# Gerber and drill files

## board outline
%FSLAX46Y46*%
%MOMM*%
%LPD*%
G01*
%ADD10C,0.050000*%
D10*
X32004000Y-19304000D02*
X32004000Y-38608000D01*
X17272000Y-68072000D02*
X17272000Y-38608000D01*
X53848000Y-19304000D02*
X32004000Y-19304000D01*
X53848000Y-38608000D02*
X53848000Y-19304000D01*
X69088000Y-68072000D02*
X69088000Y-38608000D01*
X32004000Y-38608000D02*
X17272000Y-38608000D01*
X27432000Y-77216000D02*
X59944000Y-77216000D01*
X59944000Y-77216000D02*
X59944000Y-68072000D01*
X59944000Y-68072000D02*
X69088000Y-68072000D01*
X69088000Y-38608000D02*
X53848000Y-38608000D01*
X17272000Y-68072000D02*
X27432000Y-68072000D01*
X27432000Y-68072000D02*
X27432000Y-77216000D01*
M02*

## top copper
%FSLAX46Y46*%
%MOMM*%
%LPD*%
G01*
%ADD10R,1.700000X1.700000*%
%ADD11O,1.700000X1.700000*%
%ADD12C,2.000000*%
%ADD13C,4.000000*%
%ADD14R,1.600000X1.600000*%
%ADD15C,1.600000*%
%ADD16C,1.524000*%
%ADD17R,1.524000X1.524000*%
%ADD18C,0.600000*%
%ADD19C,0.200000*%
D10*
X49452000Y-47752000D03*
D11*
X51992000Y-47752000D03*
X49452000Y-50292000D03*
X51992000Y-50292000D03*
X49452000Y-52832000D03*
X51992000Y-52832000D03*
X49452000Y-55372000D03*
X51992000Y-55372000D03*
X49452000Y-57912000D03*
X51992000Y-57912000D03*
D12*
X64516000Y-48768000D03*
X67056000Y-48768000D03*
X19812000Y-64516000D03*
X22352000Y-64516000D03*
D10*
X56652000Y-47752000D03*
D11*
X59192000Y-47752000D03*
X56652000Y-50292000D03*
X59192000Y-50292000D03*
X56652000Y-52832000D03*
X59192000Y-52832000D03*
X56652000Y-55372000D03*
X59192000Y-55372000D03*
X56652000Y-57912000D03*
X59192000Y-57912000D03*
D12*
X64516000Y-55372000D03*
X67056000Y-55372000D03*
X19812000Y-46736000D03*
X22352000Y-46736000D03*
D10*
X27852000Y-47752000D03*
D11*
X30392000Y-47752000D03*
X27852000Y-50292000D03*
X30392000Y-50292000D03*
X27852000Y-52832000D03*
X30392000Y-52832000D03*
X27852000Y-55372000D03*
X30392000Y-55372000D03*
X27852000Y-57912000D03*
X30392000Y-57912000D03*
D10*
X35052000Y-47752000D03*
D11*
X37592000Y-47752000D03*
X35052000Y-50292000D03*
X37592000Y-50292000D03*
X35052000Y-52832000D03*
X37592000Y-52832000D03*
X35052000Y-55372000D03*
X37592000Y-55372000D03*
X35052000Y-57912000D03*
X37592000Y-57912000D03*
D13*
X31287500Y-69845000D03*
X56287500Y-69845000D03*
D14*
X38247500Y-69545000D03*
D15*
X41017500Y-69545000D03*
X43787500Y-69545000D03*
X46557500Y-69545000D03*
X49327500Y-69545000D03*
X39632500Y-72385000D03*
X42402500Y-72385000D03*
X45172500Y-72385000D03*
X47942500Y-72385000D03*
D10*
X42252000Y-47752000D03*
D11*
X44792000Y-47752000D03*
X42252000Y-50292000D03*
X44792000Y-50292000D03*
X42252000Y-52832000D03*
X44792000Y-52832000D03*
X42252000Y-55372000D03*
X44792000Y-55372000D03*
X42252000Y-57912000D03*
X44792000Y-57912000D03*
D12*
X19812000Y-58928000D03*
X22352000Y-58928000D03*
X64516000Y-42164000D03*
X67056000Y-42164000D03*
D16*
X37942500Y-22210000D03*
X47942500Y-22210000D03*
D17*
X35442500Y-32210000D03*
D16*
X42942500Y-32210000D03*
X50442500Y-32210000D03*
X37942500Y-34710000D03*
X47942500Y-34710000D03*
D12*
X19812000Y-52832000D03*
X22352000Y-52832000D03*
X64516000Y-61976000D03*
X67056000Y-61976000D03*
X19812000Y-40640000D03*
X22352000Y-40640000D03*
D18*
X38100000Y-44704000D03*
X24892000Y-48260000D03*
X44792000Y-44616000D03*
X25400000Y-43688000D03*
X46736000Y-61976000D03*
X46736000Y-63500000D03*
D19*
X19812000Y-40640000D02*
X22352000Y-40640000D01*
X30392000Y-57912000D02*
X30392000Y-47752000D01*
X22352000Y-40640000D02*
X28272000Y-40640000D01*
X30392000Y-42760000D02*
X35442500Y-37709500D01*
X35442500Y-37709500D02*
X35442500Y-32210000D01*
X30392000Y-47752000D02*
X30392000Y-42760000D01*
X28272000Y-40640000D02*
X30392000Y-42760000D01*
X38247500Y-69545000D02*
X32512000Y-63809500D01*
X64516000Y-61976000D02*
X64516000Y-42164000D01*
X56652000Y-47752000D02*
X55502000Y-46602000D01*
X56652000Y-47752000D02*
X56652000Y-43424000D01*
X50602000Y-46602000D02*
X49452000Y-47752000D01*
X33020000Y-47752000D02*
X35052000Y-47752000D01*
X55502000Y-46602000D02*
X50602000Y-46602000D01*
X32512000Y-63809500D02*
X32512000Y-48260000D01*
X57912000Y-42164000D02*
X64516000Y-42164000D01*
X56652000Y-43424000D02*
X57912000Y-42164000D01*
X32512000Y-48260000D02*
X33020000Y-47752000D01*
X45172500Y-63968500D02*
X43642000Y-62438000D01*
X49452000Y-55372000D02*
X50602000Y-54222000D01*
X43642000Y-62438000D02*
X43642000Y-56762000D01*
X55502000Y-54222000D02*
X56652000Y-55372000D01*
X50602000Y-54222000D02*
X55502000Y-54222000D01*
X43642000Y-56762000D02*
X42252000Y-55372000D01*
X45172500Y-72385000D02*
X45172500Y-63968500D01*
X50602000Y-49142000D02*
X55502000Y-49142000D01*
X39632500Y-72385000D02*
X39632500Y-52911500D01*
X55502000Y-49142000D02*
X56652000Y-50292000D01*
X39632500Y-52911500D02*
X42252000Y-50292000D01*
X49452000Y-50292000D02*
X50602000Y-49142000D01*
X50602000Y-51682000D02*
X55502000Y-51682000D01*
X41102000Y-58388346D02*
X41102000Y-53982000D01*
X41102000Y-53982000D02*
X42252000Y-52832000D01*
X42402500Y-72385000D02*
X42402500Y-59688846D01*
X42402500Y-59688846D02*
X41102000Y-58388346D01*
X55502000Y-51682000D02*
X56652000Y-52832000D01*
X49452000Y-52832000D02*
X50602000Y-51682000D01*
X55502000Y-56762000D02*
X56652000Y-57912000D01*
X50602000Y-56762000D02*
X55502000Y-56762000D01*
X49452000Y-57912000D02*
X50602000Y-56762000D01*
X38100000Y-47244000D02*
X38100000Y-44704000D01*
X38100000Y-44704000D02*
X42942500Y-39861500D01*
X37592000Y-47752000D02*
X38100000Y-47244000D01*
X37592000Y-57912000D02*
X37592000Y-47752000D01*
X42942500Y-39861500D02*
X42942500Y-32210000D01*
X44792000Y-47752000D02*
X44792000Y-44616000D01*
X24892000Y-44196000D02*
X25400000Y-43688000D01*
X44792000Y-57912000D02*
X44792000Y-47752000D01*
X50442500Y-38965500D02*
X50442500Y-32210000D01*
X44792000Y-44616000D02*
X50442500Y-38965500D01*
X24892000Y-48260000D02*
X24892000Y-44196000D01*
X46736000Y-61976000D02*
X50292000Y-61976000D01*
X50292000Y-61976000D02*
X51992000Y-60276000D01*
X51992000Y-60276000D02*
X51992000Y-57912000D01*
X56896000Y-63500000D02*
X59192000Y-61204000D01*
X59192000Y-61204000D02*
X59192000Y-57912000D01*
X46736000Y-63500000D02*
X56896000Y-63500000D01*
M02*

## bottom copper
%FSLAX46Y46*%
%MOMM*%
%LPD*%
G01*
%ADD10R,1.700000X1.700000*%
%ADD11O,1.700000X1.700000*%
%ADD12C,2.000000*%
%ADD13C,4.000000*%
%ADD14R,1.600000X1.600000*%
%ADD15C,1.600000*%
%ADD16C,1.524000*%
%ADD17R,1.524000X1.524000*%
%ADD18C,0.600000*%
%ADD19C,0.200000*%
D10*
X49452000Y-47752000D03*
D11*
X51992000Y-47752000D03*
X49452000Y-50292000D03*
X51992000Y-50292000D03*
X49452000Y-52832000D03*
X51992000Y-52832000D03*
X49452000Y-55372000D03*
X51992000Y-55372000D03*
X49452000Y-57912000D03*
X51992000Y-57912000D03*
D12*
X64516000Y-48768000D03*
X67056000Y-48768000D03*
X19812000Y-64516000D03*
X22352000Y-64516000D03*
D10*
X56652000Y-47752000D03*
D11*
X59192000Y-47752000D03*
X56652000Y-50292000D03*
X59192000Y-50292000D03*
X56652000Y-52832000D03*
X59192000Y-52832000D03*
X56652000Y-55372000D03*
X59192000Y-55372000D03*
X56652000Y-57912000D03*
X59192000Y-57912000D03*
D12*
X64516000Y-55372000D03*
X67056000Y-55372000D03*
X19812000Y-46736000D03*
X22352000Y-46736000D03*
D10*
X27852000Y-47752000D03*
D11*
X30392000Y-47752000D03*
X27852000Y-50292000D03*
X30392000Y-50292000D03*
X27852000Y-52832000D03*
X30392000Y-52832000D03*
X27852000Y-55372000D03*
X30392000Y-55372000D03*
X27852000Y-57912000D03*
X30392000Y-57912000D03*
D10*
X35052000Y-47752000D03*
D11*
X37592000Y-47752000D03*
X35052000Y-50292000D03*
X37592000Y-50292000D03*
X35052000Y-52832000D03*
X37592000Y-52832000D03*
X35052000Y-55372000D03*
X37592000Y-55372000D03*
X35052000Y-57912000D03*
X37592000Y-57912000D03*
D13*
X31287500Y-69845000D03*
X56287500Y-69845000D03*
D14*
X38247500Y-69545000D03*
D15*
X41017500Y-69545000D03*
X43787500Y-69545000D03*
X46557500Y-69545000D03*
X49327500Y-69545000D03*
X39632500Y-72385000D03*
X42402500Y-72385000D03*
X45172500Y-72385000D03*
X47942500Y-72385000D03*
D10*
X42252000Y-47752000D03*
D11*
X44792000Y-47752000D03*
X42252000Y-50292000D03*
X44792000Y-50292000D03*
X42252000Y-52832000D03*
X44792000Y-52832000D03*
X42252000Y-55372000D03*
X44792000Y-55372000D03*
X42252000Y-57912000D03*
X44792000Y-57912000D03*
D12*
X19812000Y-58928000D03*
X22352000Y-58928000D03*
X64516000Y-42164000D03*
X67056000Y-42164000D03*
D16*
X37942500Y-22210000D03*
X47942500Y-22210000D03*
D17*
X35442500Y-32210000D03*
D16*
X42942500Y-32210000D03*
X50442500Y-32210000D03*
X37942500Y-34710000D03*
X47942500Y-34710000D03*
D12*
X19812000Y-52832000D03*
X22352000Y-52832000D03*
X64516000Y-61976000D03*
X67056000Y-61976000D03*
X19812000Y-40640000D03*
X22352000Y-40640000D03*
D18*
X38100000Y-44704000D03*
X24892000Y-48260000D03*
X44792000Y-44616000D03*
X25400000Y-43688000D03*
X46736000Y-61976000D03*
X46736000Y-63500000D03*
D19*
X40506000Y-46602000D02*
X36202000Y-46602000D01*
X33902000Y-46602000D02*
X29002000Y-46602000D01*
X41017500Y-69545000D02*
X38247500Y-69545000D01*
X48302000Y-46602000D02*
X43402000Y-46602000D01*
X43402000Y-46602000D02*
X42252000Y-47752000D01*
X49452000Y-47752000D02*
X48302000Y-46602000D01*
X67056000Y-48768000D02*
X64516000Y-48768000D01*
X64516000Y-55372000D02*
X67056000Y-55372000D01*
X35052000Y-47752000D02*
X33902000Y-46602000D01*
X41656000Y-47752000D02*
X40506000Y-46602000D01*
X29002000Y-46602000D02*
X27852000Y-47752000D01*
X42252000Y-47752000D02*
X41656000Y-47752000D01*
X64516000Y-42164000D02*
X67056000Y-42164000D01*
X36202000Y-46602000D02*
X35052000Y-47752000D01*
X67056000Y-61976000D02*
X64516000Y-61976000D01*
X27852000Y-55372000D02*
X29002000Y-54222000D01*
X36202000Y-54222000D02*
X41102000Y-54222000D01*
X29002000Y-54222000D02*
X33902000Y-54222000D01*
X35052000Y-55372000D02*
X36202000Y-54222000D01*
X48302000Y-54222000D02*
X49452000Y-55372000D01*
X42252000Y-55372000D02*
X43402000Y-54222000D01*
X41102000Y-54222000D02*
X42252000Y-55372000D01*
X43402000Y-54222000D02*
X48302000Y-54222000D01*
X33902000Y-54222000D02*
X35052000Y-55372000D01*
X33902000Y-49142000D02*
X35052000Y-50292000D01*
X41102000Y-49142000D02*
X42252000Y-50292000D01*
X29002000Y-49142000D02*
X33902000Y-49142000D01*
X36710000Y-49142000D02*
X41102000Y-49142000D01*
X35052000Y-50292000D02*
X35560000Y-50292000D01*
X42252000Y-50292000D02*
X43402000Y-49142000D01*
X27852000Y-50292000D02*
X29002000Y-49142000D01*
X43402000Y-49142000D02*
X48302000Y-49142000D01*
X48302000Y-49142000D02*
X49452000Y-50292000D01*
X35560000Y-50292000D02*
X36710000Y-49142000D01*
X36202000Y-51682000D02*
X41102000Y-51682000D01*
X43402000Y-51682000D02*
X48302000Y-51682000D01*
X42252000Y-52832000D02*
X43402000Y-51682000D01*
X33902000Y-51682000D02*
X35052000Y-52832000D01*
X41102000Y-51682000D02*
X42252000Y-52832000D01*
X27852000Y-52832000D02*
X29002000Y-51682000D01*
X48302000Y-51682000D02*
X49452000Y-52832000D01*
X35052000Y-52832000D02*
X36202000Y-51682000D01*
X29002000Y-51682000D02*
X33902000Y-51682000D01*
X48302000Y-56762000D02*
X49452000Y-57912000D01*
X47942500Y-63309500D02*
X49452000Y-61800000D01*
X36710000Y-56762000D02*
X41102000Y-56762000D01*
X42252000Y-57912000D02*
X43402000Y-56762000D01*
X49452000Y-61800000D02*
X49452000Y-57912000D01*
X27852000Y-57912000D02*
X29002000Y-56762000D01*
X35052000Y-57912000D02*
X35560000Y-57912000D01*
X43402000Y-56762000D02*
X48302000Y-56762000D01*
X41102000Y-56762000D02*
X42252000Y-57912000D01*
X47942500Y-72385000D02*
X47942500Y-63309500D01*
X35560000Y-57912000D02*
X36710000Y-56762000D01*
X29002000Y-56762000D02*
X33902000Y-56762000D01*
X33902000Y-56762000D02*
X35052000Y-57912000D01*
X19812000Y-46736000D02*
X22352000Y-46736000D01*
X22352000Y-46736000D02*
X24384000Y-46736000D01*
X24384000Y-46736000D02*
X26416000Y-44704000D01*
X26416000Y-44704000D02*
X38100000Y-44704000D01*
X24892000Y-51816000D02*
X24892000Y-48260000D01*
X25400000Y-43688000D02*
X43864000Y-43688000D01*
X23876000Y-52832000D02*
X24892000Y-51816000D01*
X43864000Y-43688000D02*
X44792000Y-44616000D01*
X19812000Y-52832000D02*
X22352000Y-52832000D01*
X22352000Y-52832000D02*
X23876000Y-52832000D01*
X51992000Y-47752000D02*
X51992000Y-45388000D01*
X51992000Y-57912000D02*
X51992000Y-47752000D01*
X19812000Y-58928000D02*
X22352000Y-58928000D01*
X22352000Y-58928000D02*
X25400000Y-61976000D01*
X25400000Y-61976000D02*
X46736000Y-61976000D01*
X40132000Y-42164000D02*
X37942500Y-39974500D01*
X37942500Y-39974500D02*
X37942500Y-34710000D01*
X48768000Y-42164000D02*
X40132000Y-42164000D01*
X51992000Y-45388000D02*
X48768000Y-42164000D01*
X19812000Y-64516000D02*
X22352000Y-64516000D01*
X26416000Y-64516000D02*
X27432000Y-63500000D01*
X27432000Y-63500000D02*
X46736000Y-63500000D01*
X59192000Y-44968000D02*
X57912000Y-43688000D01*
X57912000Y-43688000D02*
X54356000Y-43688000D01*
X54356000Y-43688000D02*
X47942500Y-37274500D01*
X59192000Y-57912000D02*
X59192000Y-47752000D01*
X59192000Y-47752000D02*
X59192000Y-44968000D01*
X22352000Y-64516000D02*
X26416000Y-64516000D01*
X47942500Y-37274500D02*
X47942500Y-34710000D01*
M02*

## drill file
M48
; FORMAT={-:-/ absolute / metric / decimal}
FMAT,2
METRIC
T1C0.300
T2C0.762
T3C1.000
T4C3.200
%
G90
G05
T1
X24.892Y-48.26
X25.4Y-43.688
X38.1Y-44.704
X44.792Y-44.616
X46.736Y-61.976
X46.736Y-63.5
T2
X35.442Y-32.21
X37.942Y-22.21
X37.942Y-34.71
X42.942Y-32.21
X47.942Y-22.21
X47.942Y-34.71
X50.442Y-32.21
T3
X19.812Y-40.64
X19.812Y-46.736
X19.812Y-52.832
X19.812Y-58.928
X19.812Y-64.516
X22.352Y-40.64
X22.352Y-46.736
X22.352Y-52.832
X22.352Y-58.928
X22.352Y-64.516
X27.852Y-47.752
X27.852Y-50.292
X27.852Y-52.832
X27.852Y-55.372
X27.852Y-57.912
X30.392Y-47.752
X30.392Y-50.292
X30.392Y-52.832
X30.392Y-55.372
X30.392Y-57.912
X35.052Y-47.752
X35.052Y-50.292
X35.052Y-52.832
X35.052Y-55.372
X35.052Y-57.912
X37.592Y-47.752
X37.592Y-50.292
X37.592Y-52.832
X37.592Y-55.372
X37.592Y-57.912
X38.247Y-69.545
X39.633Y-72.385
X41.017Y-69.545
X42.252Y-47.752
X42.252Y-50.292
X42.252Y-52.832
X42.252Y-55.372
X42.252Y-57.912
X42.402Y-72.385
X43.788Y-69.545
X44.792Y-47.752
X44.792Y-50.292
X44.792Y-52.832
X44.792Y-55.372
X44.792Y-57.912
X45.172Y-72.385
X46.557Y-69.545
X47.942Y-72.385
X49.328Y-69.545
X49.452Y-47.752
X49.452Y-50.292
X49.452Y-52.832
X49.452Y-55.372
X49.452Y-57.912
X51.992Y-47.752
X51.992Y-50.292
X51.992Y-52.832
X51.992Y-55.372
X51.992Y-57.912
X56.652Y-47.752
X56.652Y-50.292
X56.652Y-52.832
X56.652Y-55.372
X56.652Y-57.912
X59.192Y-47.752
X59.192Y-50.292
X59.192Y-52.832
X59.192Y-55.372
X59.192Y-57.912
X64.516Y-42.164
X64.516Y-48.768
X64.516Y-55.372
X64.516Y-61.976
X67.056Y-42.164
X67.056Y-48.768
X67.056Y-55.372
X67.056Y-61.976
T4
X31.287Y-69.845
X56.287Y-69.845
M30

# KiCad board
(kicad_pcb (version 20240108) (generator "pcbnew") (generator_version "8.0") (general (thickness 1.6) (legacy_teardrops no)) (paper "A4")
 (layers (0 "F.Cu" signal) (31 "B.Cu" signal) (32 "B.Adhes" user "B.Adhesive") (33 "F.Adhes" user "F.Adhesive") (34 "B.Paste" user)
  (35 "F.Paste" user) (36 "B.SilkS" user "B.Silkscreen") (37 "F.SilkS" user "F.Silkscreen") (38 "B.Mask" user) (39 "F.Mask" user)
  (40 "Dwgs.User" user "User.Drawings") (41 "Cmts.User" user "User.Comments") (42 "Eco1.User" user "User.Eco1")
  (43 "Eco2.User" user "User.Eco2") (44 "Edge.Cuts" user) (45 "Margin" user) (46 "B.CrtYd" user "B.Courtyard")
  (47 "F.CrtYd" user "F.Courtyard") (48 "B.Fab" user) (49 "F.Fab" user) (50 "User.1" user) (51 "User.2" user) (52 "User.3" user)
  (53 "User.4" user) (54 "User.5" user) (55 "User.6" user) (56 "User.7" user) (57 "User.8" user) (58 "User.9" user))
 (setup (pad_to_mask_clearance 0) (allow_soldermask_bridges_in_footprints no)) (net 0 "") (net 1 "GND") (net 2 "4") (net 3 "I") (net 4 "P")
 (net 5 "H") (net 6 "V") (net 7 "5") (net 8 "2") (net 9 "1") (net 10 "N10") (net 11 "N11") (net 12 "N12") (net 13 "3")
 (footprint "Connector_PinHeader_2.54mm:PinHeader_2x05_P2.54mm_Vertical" (layer "F.Cu") (at 49.452 47.752)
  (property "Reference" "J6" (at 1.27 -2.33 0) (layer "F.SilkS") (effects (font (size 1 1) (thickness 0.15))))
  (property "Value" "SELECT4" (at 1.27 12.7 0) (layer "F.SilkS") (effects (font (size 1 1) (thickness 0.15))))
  (pad "1" thru_hole rect (at 0 0) (size 1.7 1.7) (drill 1) (layers "*.Cu" "*.Mask") (remove_unused_layers no) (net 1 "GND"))
  (pad "2" thru_hole oval (at 2.54 0) (size 1.7 1.7) (drill 1) (layers "*.Cu" "*.Mask") (remove_unused_layers no) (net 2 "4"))
  (pad "3" thru_hole oval (at 0 2.54) (size 1.7 1.7) (drill 1) (layers "*.Cu" "*.Mask") (remove_unused_layers no) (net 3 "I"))
  (pad "4" thru_hole oval (at 2.54 2.54) (size 1.7 1.7) (drill 1) (layers "*.Cu" "*.Mask") (remove_unused_layers no) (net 2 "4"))
  (pad "5" thru_hole oval (at 0 5.08) (size 1.7 1.7) (drill 1) (layers "*.Cu" "*.Mask") (remove_unused_layers no) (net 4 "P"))
  (pad "6" thru_hole oval (at 2.54 5.08) (size 1.7 1.7) (drill 1) (layers "*.Cu" "*.Mask") (remove_unused_layers no) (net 2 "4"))
  (pad "7" thru_hole oval (at 0 7.62) (size 1.7 1.7) (drill 1) (layers "*.Cu" "*.Mask") (remove_unused_layers no) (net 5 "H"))
  (pad "8" thru_hole oval (at 2.54 7.62) (size 1.7 1.7) (drill 1) (layers "*.Cu" "*.Mask") (remove_unused_layers no) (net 2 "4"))
  (pad "9" thru_hole oval (at 0 10.16) (size 1.7 1.7) (drill 1) (layers "*.Cu" "*.Mask") (remove_unused_layers no) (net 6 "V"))
  (pad "10" thru_hole oval (at 2.54 10.16) (size 1.7 1.7) (drill 1) (layers "*.Cu" "*.Mask") (remove_unused_layers no) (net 2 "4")))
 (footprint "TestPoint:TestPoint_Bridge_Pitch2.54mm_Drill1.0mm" (layer "F.Cu") (at 64.516 48.768)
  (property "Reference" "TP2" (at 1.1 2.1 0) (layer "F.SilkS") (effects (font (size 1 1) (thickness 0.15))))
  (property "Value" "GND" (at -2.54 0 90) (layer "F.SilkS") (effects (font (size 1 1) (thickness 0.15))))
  (pad "1" thru_hole circle (at 0 0) (size 2 2) (drill 1) (layers "*.Cu" "*.Mask") (remove_unused_layers no) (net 1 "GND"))
  (pad "1" thru_hole circle (at 2.54 0) (size 2 2) (drill 1) (layers "*.Cu" "*.Mask") (remove_unused_layers no) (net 1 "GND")))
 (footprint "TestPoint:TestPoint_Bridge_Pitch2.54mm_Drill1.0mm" (layer "F.Cu") (at 19.812 64.516)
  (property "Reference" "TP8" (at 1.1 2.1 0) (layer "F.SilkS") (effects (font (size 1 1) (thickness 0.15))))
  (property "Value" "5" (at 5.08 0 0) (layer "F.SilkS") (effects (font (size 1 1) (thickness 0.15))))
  (pad "1" thru_hole circle (at 0 0) (size 2 2) (drill 1) (layers "*.Cu" "*.Mask") (remove_unused_layers no) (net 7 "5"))
  (pad "1" thru_hole circle (at 2.54 0) (size 2 2) (drill 1) (layers "*.Cu" "*.Mask") (remove_unused_layers no) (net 7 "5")))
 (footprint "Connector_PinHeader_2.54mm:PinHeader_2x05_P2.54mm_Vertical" (layer "F.Cu") (at 56.652 47.752)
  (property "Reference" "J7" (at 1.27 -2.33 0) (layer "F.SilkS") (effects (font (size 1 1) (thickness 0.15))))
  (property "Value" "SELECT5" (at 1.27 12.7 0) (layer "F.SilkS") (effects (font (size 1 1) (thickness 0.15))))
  (pad "1" thru_hole rect (at 0 0) (size 1.7 1.7) (drill 1) (layers "*.Cu" "*.Mask") (remove_unused_layers no) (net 1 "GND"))
  (pad "2" thru_hole oval (at 2.54 0) (size 1.7 1.7) (drill 1) (layers "*.Cu" "*.Mask") (remove_unused_layers no) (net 7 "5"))
  (pad "3" thru_hole oval (at 0 2.54) (size 1.7 1.7) (drill 1) (layers "*.Cu" "*.Mask") (remove_unused_layers no) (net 3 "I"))
  (pad "4" thru_hole oval (at 2.54 2.54) (size 1.7 1.7) (drill 1) (layers "*.Cu" "*.Mask") (remove_unused_layers no) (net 7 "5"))
  (pad "5" thru_hole oval (at 0 5.08) (size 1.7 1.7) (drill 1) (layers "*.Cu" "*.Mask") (remove_unused_layers no) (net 4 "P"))
  (pad "6" thru_hole oval (at 2.54 5.08) (size 1.7 1.7) (drill 1) (layers "*.Cu" "*.Mask") (remove_unused_layers no) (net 7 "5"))
  (pad "7" thru_hole oval (at 0 7.62) (size 1.7 1.7) (drill 1) (layers "*.Cu" "*.Mask") (remove_unused_layers no) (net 5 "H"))
  (pad "8" thru_hole oval (at 2.54 7.62) (size 1.7 1.7) (drill 1) (layers "*.Cu" "*.Mask") (remove_unused_layers no) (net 7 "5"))
  (pad "9" thru_hole oval (at 0 10.16) (size 1.7 1.7) (drill 1) (layers "*.Cu" "*.Mask") (remove_unused_layers no) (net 6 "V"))
  (pad "10" thru_hole oval (at 2.54 10.16) (size 1.7 1.7) (drill 1) (layers "*.Cu" "*.Mask") (remove_unused_layers no) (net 7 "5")))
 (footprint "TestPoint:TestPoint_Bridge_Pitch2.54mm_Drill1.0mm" (layer "F.Cu") (at 64.516 55.372)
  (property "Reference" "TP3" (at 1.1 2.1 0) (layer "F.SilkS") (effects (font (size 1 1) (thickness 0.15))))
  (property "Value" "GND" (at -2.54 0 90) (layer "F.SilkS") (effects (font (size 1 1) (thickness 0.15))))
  (pad "1" thru_hole circle (at 0 0) (size 2 2) (drill 1) (layers "*.Cu" "*.Mask") (remove_unused_layers no) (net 1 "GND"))
  (pad "1" thru_hole circle (at 2.54 0) (size 2 2) (drill 1) (layers "*.Cu" "*.Mask") (remove_unused_layers no) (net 1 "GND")))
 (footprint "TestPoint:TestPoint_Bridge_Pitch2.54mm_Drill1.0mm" (layer "F.Cu") (at 19.812 46.736)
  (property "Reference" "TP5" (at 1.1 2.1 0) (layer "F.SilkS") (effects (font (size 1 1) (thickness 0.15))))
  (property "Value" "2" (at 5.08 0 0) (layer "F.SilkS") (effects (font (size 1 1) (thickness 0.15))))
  (pad "1" thru_hole circle (at 0 0) (size 2 2) (drill 1) (layers "*.Cu" "*.Mask") (remove_unused_layers no) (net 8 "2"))
  (pad "1" thru_hole circle (at 2.54 0) (size 2 2) (drill 1) (layers "*.Cu" "*.Mask") (remove_unused_layers no) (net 8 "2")))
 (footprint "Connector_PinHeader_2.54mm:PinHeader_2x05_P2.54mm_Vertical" (layer "F.Cu") (at 27.852 47.752)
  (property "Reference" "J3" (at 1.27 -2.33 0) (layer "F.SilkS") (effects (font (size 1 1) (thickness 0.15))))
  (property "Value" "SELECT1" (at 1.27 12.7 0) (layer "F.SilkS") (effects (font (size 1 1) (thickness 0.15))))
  (pad "1" thru_hole rect (at 0 0) (size 1.7 1.7) (drill 1) (layers "*.Cu" "*.Mask") (remove_unused_layers no) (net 1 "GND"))
  (pad "2" thru_hole oval (at 2.54 0) (size 1.7 1.7) (drill 1) (layers "*.Cu" "*.Mask") (remove_unused_layers no) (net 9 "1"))
  (pad "3" thru_hole oval (at 0 2.54) (size 1.7 1.7) (drill 1) (layers "*.Cu" "*.Mask") (remove_unused_layers no) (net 3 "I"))
  (pad "4" thru_hole oval (at 2.54 2.54) (size 1.7 1.7) (drill 1) (layers "*.Cu" "*.Mask") (remove_unused_layers no) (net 9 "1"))
  (pad "5" thru_hole oval (at 0 5.08) (size 1.7 1.7) (drill 1) (layers "*.Cu" "*.Mask") (remove_unused_layers no) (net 4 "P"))
  (pad "6" thru_hole oval (at 2.54 5.08) (size 1.7 1.7) (drill 1) (layers "*.Cu" "*.Mask") (remove_unused_layers no) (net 9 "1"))
  (pad "7" thru_hole oval (at 0 7.62) (size 1.7 1.7) (drill 1) (layers "*.Cu" "*.Mask") (remove_unused_layers no) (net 5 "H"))
  (pad "8" thru_hole oval (at 2.54 7.62) (size 1.7 1.7) (drill 1) (layers "*.Cu" "*.Mask") (remove_unused_layers no) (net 9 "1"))
  (pad "9" thru_hole oval (at 0 10.16) (size 1.7 1.7) (drill 1) (layers "*.Cu" "*.Mask") (remove_unused_layers no) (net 6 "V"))
  (pad "10" thru_hole oval (at 2.54 10.16) (size 1.7 1.7) (drill 1) (layers "*.Cu" "*.Mask") (remove_unused_layers no) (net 9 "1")))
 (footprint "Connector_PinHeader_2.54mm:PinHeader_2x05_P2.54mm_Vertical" (layer "F.Cu") (at 35.052 47.752)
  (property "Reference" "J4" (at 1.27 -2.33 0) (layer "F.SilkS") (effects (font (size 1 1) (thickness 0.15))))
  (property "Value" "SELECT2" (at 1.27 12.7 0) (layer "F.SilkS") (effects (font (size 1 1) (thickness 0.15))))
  (pad "1" thru_hole rect (at 0 0) (size 1.7 1.7) (drill 1) (layers "*.Cu" "*.Mask") (remove_unused_layers no) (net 1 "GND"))
  (pad "2" thru_hole oval (at 2.54 0) (size 1.7 1.7) (drill 1) (layers "*.Cu" "*.Mask") (remove_unused_layers no) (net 8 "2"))
  (pad "3" thru_hole oval (at 0 2.54) (size 1.7 1.7) (drill 1) (layers "*.Cu" "*.Mask") (remove_unused_layers no) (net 3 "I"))
  (pad "4" thru_hole oval (at 2.54 2.54) (size 1.7 1.7) (drill 1) (layers "*.Cu" "*.Mask") (remove_unused_layers no) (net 8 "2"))
  (pad "5" thru_hole oval (at 0 5.08) (size 1.7 1.7) (drill 1) (layers "*.Cu" "*.Mask") (remove_unused_layers no) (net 4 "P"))
  (pad "6" thru_hole oval (at 2.54 5.08) (size 1.7 1.7) (drill 1) (layers "*.Cu" "*.Mask") (remove_unused_layers no) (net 8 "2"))
  (pad "7" thru_hole oval (at 0 7.62) (size 1.7 1.7) (drill 1) (layers "*.Cu" "*.Mask") (remove_unused_layers no) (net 5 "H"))
  (pad "8" thru_hole oval (at 2.54 7.62) (size 1.7 1.7) (drill 1) (layers "*.Cu" "*.Mask") (remove_unused_layers no) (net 8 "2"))
  (pad "9" thru_hole oval (at 0 10.16) (size 1.7 1.7) (drill 1) (layers "*.Cu" "*.Mask") (remove_unused_layers no) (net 6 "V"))
  (pad "10" thru_hole oval (at 2.54 10.16) (size 1.7 1.7) (drill 1) (layers "*.Cu" "*.Mask") (remove_unused_layers no) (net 8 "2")))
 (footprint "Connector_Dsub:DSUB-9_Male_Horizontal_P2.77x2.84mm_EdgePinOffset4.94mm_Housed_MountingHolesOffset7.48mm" (layer "F.Cu")
  (at 38.2475 69.545)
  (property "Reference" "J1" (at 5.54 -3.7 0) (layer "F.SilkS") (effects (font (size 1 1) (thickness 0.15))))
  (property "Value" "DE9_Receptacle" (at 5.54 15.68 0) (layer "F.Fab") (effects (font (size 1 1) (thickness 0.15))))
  (pad "0" thru_hole circle (at -6.96 0.3) (size 4 4) (drill 3.2) (layers "*.Cu" "*.Mask") (remove_unused_layers no))
  (pad "0" thru_hole circle (at 18.04 0.3) (size 4 4) (drill 3.2) (layers "*.Cu" "*.Mask") (remove_unused_layers no))
  (pad "1" thru_hole rect (at 0 0) (size 1.6 1.6) (drill 1) (layers "*.Cu" "*.Mask") (remove_unused_layers no) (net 1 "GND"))
  (pad "2" thru_hole circle (at 2.77 0) (size 1.6 1.6) (drill 1) (layers "*.Cu" "*.Mask") (remove_unused_layers no) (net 1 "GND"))
  (pad "3" thru_hole circle (at 5.54 0) (size 1.6 1.6) (drill 1) (layers "*.Cu" "*.Mask") (remove_unused_layers no) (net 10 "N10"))
  (pad "4" thru_hole circle (at 8.31 0) (size 1.6 1.6) (drill 1) (layers "*.Cu" "*.Mask") (remove_unused_layers no) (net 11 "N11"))
  (pad "5" thru_hole circle (at 11.08 0) (size 1.6 1.6) (drill 1) (layers "*.Cu" "*.Mask") (remove_unused_layers no) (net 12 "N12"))
  (pad "6" thru_hole circle (at 1.385 2.84) (size 1.6 1.6) (drill 1) (layers "*.Cu" "*.Mask") (remove_unused_layers no) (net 3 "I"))
  (pad "7" thru_hole circle (at 4.155 2.84) (size 1.6 1.6) (drill 1) (layers "*.Cu" "*.Mask") (remove_unused_layers no) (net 4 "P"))
  (pad "8" thru_hole circle (at 6.925 2.84) (size 1.6 1.6) (drill 1) (layers "*.Cu" "*.Mask") (remove_unused_layers no) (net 5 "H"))
  (pad "9" thru_hole circle (at 9.695 2.84) (size 1.6 1.6) (drill 1) (layers "*.Cu" "*.Mask") (remove_unused_layers no) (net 6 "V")))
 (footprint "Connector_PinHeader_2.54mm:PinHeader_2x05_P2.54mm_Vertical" (layer "F.Cu") (at 42.252 47.752)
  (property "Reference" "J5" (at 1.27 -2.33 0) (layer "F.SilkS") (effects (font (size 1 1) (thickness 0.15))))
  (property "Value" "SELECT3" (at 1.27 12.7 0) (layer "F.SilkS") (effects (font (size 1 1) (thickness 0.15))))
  (pad "1" thru_hole rect (at 0 0) (size 1.7 1.7) (drill 1) (layers "*.Cu" "*.Mask") (remove_unused_layers no) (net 1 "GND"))
  (pad "2" thru_hole oval (at 2.54 0) (size 1.7 1.7) (drill 1) (layers "*.Cu" "*.Mask") (remove_unused_layers no) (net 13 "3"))
  (pad "3" thru_hole oval (at 0 2.54) (size 1.7 1.7) (drill 1) (layers "*.Cu" "*.Mask") (remove_unused_layers no) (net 3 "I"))
  (pad "4" thru_hole oval (at 2.54 2.54) (size 1.7 1.7) (drill 1) (layers "*.Cu" "*.Mask") (remove_unused_layers no) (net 13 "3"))
  (pad "5" thru_hole oval (at 0 5.08) (size 1.7 1.7) (drill 1) (layers "*.Cu" "*.Mask") (remove_unused_layers no) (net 4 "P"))
  (pad "6" thru_hole oval (at 2.54 5.08) (size 1.7 1.7) (drill 1) (layers "*.Cu" "*.Mask") (remove_unused_layers no) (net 13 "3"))
  (pad "7" thru_hole oval (at 0 7.62) (size 1.7 1.7) (drill 1) (layers "*.Cu" "*.Mask") (remove_unused_layers no) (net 5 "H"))
  (pad "8" thru_hole oval (at 2.54 7.62) (size 1.7 1.7) (drill 1) (layers "*.Cu" "*.Mask") (remove_unused_layers no) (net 13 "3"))
  (pad "9" thru_hole oval (at 0 10.16) (size 1.7 1.7) (drill 1) (layers "*.Cu" "*.Mask") (remove_unused_layers no) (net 6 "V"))
  (pad "10" thru_hole oval (at 2.54 10.16) (size 1.7 1.7) (drill 1) (layers "*.Cu" "*.Mask") (remove_unused_layers no) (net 13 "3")))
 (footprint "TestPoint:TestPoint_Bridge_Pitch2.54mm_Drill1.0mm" (layer "F.Cu") (at 19.812 58.928)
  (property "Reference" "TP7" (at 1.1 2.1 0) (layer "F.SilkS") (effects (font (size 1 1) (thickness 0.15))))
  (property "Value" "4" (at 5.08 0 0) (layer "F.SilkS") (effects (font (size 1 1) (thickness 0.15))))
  (pad "1" thru_hole circle (at 0 0) (size 2 2) (drill 1) (layers "*.Cu" "*.Mask") (remove_unused_layers no) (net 2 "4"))
  (pad "1" thru_hole circle (at 2.54 0) (size 2 2) (drill 1) (layers "*.Cu" "*.Mask") (remove_unused_layers no) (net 2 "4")))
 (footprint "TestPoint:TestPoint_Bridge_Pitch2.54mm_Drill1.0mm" (layer "F.Cu") (at 64.516 42.164)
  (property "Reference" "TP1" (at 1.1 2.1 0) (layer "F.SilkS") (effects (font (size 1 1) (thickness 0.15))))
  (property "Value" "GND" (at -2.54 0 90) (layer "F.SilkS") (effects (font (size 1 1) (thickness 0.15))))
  (pad "1" thru_hole circle (at 0 0) (size 2 2) (drill 1) (layers "*.Cu" "*.Mask") (remove_unused_layers no) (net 1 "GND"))
  (pad "1" thru_hole circle (at 2.54 0) (size 2 2) (drill 1) (layers "*.Cu" "*.Mask") (remove_unused_layers no) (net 1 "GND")))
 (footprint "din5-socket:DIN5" (layer "F.Cu") (at 42.9425 32.21)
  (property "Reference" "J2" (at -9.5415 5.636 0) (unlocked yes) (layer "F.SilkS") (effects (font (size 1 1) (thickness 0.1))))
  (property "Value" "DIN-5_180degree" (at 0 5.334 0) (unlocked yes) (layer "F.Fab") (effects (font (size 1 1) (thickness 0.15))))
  (pad "" thru_hole circle (at -5 -10) (size 1.524 1.524) (drill 0.762) (layers "*.Cu" "*.Mask") (remove_unused_layers no))
  (pad "" thru_hole circle (at 5 -10) (size 1.524 1.524) (drill 0.762) (layers "*.Cu" "*.Mask") (remove_unused_layers no))
  (pad "1" thru_hole rect (at -7.5 0) (size 1.524 1.524) (drill 0.762) (layers "*.Cu" "*.Mask") (remove_unused_layers no) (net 9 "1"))
  (pad "2" thru_hole circle (at 0 0) (size 1.524 1.524) (drill 0.762) (layers "*.Cu" "*.Mask") (remove_unused_layers no) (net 8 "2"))
  (pad "3" thru_hole circle (at 7.5 0) (size 1.524 1.524) (drill 0.762) (layers "*.Cu" "*.Mask") (remove_unused_layers no) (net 13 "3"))
  (pad "4" thru_hole circle (at -5 2.5) (size 1.524 1.524) (drill 0.762) (layers "*.Cu" "*.Mask") (remove_unused_layers no) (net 2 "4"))
  (pad "5" thru_hole circle (at 5 2.5) (size 1.524 1.524) (drill 0.762) (layers "*.Cu" "*.Mask") (remove_unused_layers no) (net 7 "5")))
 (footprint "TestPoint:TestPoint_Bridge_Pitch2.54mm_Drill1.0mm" (layer "F.Cu") (at 19.812 52.832)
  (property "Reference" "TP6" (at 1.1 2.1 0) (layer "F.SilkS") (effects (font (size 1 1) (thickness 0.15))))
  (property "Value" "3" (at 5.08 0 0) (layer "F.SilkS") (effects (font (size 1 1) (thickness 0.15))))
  (pad "1" thru_hole circle (at 0 0) (size 2 2) (drill 1) (layers "*.Cu" "*.Mask") (remove_unused_layers no) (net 13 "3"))
  (pad "1" thru_hole circle (at 2.54 0) (size 2 2) (drill 1) (layers "*.Cu" "*.Mask") (remove_unused_layers no) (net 13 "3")))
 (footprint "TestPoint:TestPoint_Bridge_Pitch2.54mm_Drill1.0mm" (layer "F.Cu") (at 64.516 61.976)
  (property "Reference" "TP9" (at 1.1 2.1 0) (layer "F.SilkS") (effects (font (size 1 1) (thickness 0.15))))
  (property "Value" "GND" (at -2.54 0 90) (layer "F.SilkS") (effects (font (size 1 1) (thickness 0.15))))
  (pad "1" thru_hole circle (at 0 0) (size 2 2) (drill 1) (layers "*.Cu" "*.Mask") (remove_unused_layers no) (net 1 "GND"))
  (pad "1" thru_hole circle (at 2.54 0) (size 2 2) (drill 1) (layers "*.Cu" "*.Mask") (remove_unused_layers no) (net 1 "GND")))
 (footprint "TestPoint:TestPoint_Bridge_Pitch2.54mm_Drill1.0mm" (layer "F.Cu") (at 19.812 40.64)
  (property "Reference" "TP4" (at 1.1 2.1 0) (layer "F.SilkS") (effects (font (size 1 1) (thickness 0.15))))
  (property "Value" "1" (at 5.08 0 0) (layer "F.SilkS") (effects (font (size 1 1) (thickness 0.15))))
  (pad "1" thru_hole circle (at 0 0) (size 2 2) (drill 1) (layers "*.Cu" "*.Mask") (remove_unused_layers no) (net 9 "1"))
  (pad "1" thru_hole circle (at 2.54 0) (size 2 2) (drill 1) (layers "*.Cu" "*.Mask") (remove_unused_layers no) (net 9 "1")))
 (gr_line (start 32.004 19.304) (end 32.004 38.608) (stroke (width 0.05) (type default)) (layer "Edge.Cuts"))
 (gr_line (start 17.272 68.072) (end 17.272 38.608) (stroke (width 0.05) (type default)) (layer "Edge.Cuts"))
 (gr_line (start 53.848 19.304) (end 32.004 19.304) (stroke (width 0.05) (type default)) (layer "Edge.Cuts"))
 (gr_line (start 53.848 38.608) (end 53.848 19.304) (stroke (width 0.05) (type default)) (layer "Edge.Cuts"))
 (gr_line (start 69.088 68.072) (end 69.088 38.608) (stroke (width 0.05) (type default)) (layer "Edge.Cuts"))
 (gr_line (start 32.004 38.608) (end 17.272 38.608) (stroke (width 0.05) (type default)) (layer "Edge.Cuts"))
 (gr_line (start 27.432 77.216) (end 59.944 77.216) (stroke (width 0.05) (type default)) (layer "Edge.Cuts"))
 (gr_line (start 59.944 77.216) (end 59.944 68.072) (stroke (width 0.05) (type default)) (layer "Edge.Cuts"))
 (gr_line (start 59.944 68.072) (end 69.088 68.072) (stroke (width 0.05) (type default)) (layer "Edge.Cuts"))
 (gr_line (start 69.088 38.608) (end 53.848 38.608) (stroke (width 0.05) (type default)) (layer "Edge.Cuts"))
 (gr_line (start 17.272 68.072) (end 27.432 68.072) (stroke (width 0.05) (type default)) (layer "Edge.Cuts"))
 (gr_line (start 27.432 68.072) (end 27.432 77.216) (stroke (width 0.05) (type default)) (layer "Edge.Cuts"))
 (segment (start 19.812 40.64) (end 22.352 40.64) (width 0.2) (layer "F.Cu") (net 9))
 (segment (start 30.392 57.912) (end 30.392 47.752) (width 0.2) (layer "F.Cu") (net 9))
 (segment (start 22.352 40.64) (end 28.272 40.64) (width 0.2) (layer "F.Cu") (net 9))
 (segment (start 30.392 42.76) (end 35.4425 37.7095) (width 0.2) (layer "F.Cu") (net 9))
 (segment (start 35.4425 37.7095) (end 35.4425 32.21) (width 0.2) (layer "F.Cu") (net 9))
 (segment (start 30.392 47.752) (end 30.392 42.76) (width 0.2) (layer "F.Cu") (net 9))
 (segment (start 28.272 40.64) (end 30.392 42.76) (width 0.2) (layer "F.Cu") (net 9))
 (segment (start 38.2475 69.545) (end 32.512 63.8095) (width 0.2) (layer "F.Cu") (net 1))
 (segment (start 64.516 61.976) (end 64.516 42.164) (width 0.2) (layer "F.Cu") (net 1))
 (segment (start 56.652 47.752) (end 55.502 46.602) (width 0.2) (layer "F.Cu") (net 1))
 (segment (start 56.652 47.752) (end 56.652 43.424) (width 0.2) (layer "F.Cu") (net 1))
 (segment (start 50.602 46.602) (end 49.452 47.752) (width 0.2) (layer "F.Cu") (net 1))
 (segment (start 33.02 47.752) (end 35.052 47.752) (width 0.2) (layer "F.Cu") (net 1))
 (segment (start 55.502 46.602) (end 50.602 46.602) (width 0.2) (layer "F.Cu") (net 1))
 (segment (start 32.512 63.8095) (end 32.512 48.26) (width 0.2) (layer "F.Cu") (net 1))
 (segment (start 57.912 42.164) (end 64.516 42.164) (width 0.2) (layer "F.Cu") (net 1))
 (segment (start 56.652 43.424) (end 57.912 42.164) (width 0.2) (layer "F.Cu") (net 1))
 (segment (start 32.512 48.26) (end 33.02 47.752) (width 0.2) (layer "F.Cu") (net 1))
 (segment (start 40.506 46.602) (end 36.202 46.602) (width 0.2) (layer "B.Cu") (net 1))
 (segment (start 33.902 46.602) (end 29.002 46.602) (width 0.2) (layer "B.Cu") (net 1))
 (segment (start 41.0175 69.545) (end 38.2475 69.545) (width 0.2) (layer "B.Cu") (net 1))
 (segment (start 48.302 46.602) (end 43.402 46.602) (width 0.2) (layer "B.Cu") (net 1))
 (segment (start 43.402 46.602) (end 42.252 47.752) (width 0.2) (layer "B.Cu") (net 1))
 (segment (start 49.452 47.752) (end 48.302 46.602) (width 0.2) (layer "B.Cu") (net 1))
 (segment (start 67.056 48.768) (end 64.516 48.768) (width 0.2) (layer "B.Cu") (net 1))
 (segment (start 64.516 55.372) (end 67.056 55.372) (width 0.2) (layer "B.Cu") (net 1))
 (segment (start 35.052 47.752) (end 33.902 46.602) (width 0.2) (layer "B.Cu") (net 1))
 (segment (start 41.656 47.752) (end 40.506 46.602) (width 0.2) (layer "B.Cu") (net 1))
 (segment (start 29.002 46.602) (end 27.852 47.752) (width 0.2) (layer "B.Cu") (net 1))
 (segment (start 42.252 47.752) (end 41.656 47.752) (width 0.2) (layer "B.Cu") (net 1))
 (segment (start 64.516 42.164) (end 67.056 42.164) (width 0.2) (layer "B.Cu") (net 1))
 (segment (start 36.202 46.602) (end 35.052 47.752) (width 0.2) (layer "B.Cu") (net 1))
 (segment (start 67.056 61.976) (end 64.516 61.976) (width 0.2) (layer "B.Cu") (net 1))
 (segment (start 45.1725 63.9685) (end 43.642 62.438) (width 0.2) (layer "F.Cu") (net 5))
 (segment (start 49.452 55.372) (end 50.602 54.222) (width 0.2) (layer "F.Cu") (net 5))
 (segment (start 43.642 62.438) (end 43.642 56.762) (width 0.2) (layer "F.Cu") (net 5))
 (segment (start 55.502 54.222) (end 56.652 55.372) (width 0.2) (layer "F.Cu") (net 5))
 (segment (start 50.602 54.222) (end 55.502 54.222) (width 0.2) (layer "F.Cu") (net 5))
 (segment (start 43.642 56.762) (end 42.252 55.372) (width 0.2) (layer "F.Cu") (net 5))
 (segment (start 45.1725 72.385) (end 45.1725 63.9685) (width 0.2) (layer "F.Cu") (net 5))
 (segment (start 27.852 55.372) (end 29.002 54.222) (width 0.2) (layer "B.Cu") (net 5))
 (segment (start 36.202 54.222) (end 41.102 54.222) (width 0.2) (layer "B.Cu") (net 5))
 (segment (start 29.002 54.222) (end 33.902 54.222) (width 0.2) (layer "B.Cu") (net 5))
 (segment (start 35.052 55.372) (end 36.202 54.222) (width 0.2) (layer "B.Cu") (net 5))
 (segment (start 48.302 54.222) (end 49.452 55.372) (width 0.2) (layer "B.Cu") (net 5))
 (segment (start 42.252 55.372) (end 43.402 54.222) (width 0.2) (layer "B.Cu") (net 5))
 (segment (start 41.102 54.222) (end 42.252 55.372) (width 0.2) (layer "B.Cu") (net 5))
 (segment (start 43.402 54.222) (end 48.302 54.222) (width 0.2) (layer "B.Cu") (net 5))
 (segment (start 33.902 54.222) (end 35.052 55.372) (width 0.2) (layer "B.Cu") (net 5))
 (segment (start 50.602 49.142) (end 55.502 49.142) (width 0.2) (layer "F.Cu") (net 3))
 (segment (start 39.6325 72.385) (end 39.6325 52.9115) (width 0.2) (layer "F.Cu") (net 3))
 (segment (start 55.502 49.142) (end 56.652 50.292) (width 0.2) (layer "F.Cu") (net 3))
 (segment (start 39.6325 52.9115) (end 42.252 50.292) (width 0.2) (layer "F.Cu") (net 3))
 (segment (start 49.452 50.292) (end 50.602 49.142) (width 0.2) (layer "F.Cu") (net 3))
 (segment (start 33.902 49.142) (end 35.052 50.292) (width 0.2) (layer "B.Cu") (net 3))
 (segment (start 41.102 49.142) (end 42.252 50.292) (width 0.2) (layer "B.Cu") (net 3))
 (segment (start 29.002 49.142) (end 33.902 49.142) (width 0.2) (layer "B.Cu") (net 3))
 (segment (start 36.71 49.142) (end 41.102 49.142) (width 0.2) (layer "B.Cu") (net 3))
 (segment (start 35.052 50.292) (end 35.56 50.292) (width 0.2) (layer "B.Cu") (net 3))
 (segment (start 42.252 50.292) (end 43.402 49.142) (width 0.2) (layer "B.Cu") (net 3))
 (segment (start 27.852 50.292) (end 29.002 49.142) (width 0.2) (layer "B.Cu") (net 3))
 (segment (start 43.402 49.142) (end 48.302 49.142) (width 0.2) (layer "B.Cu") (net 3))
 (segment (start 48.302 49.142) (end 49.452 50.292) (width 0.2) (layer "B.Cu") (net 3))
 (segment (start 35.56 50.292) (end 36.71 49.142) (width 0.2) (layer "B.Cu") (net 3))
 (segment (start 50.602 51.682) (end 55.502 51.682) (width 0.2) (layer "F.Cu") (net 4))
 (segment (start 41.102 58.388346) (end 41.102 53.982) (width 0.2) (layer "F.Cu") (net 4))
 (segment (start 41.102 53.982) (end 42.252 52.832) (width 0.2) (layer "F.Cu") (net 4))
 (segment (start 42.4025 72.385) (end 42.4025 59.688846) (width 0.2) (layer "F.Cu") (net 4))
 (segment (start 42.4025 59.688846) (end 41.102 58.388346) (width 0.2) (layer "F.Cu") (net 4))
 (segment (start 55.502 51.682) (end 56.652 52.832) (width 0.2) (layer "F.Cu") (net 4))
 (segment (start 49.452 52.832) (end 50.602 51.682) (width 0.2) (layer "F.Cu") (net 4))
 (segment (start 36.202 51.682) (end 41.102 51.682) (width 0.2) (layer "B.Cu") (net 4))
 (segment (start 43.402 51.682) (end 48.302 51.682) (width 0.2) (layer "B.Cu") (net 4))
 (segment (start 42.252 52.832) (end 43.402 51.682) (width 0.2) (layer "B.Cu") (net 4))
 (segment (start 33.902 51.682) (end 35.052 52.832) (width 0.2) (layer "B.Cu") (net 4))
 (segment (start 41.102 51.682) (end 42.252 52.832) (width 0.2) (layer "B.Cu") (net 4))
 (segment (start 27.852 52.832) (end 29.002 51.682) (width 0.2) (layer "B.Cu") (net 4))
 (segment (start 48.302 51.682) (end 49.452 52.832) (width 0.2) (layer "B.Cu") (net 4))
 (segment (start 35.052 52.832) (end 36.202 51.682) (width 0.2) (layer "B.Cu") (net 4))
 (segment (start 29.002 51.682) (end 33.902 51.682) (width 0.2) (layer "B.Cu") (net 4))
 (segment (start 55.502 56.762) (end 56.652 57.912) (width 0.2) (layer "F.Cu") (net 6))
 (segment (start 50.602 56.762) (end 55.502 56.762) (width 0.2) (layer "F.Cu") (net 6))
 (segment (start 49.452 57.912) (end 50.602 56.762) (width 0.2) (layer "F.Cu") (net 6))
 (segment (start 48.302 56.762) (end 49.452 57.912) (width 0.2) (layer "B.Cu") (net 6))
 (segment (start 47.9425 63.3095) (end 49.452 61.8) (width 0.2) (layer "B.Cu") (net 6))
 (segment (start 36.71 56.762) (end 41.102 56.762) (width 0.2) (layer "B.Cu") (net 6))
 (segment (start 42.252 57.912) (end 43.402 56.762) (width 0.2) (layer "B.Cu") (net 6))
 (segment (start 49.452 61.8) (end 49.452 57.912) (width 0.2) (layer "B.Cu") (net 6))
 (segment (start 27.852 57.912) (end 29.002 56.762) (width 0.2) (layer "B.Cu") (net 6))
 (segment (start 35.052 57.912) (end 35.56 57.912) (width 0.2) (layer "B.Cu") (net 6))
 (segment (start 43.402 56.762) (end 48.302 56.762) (width 0.2) (layer "B.Cu") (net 6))
 (segment (start 41.102 56.762) (end 42.252 57.912) (width 0.2) (layer "B.Cu") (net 6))
 (segment (start 47.9425 72.385) (end 47.9425 63.3095) (width 0.2) (layer "B.Cu") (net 6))
 (segment (start 35.56 57.912) (end 36.71 56.762) (width 0.2) (layer "B.Cu") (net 6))
 (segment (start 29.002 56.762) (end 33.902 56.762) (width 0.2) (layer "B.Cu") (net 6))
 (segment (start 33.902 56.762) (end 35.052 57.912) (width 0.2) (layer "B.Cu") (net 6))
 (segment (start 38.1 47.244) (end 38.1 44.704) (width 0.2) (layer "F.Cu") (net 8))
 (segment (start 38.1 44.704) (end 42.9425 39.8615) (width 0.2) (layer "F.Cu") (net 8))
 (segment (start 37.592 47.752) (end 38.1 47.244) (width 0.2) (layer "F.Cu") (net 8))
 (segment (start 37.592 57.912) (end 37.592 47.752) (width 0.2) (layer "F.Cu") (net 8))
 (segment (start 42.9425 39.8615) (end 42.9425 32.21) (width 0.2) (layer "F.Cu") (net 8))
 (via (at 38.1 44.704) (size 0.6) (drill 0.3) (layers "F.Cu" "B.Cu") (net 8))
 (segment (start 19.812 46.736) (end 22.352 46.736) (width 0.2) (layer "B.Cu") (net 8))
 (segment (start 22.352 46.736) (end 24.384 46.736) (width 0.2) (layer "B.Cu") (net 8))
 (segment (start 24.384 46.736) (end 26.416 44.704) (width 0.2) (layer "B.Cu") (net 8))
 (segment (start 26.416 44.704) (end 38.1 44.704) (width 0.2) (layer "B.Cu") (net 8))
 (segment (start 44.792 47.752) (end 44.792 44.616) (width 0.2) (layer "F.Cu") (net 13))
 (segment (start 24.892 44.196) (end 25.4 43.688) (width 0.2) (layer "F.Cu") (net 13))
 (segment (start 44.792 57.912) (end 44.792 47.752) (width 0.2) (layer "F.Cu") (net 13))
 (segment (start 50.4425 38.9655) (end 50.4425 32.21) (width 0.2) (layer "F.Cu") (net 13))
 (segment (start 44.792 44.616) (end 50.4425 38.9655) (width 0.2) (layer "F.Cu") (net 13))
 (segment (start 24.892 48.26) (end 24.892 44.196) (width 0.2) (layer "F.Cu") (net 13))
 (via (at 24.892 48.26) (size 0.6) (drill 0.3) (layers "F.Cu" "B.Cu") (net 13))
 (via (at 44.792 44.616) (size 0.6) (drill 0.3) (layers "F.Cu" "B.Cu") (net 13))
 (via (at 25.4 43.688) (size 0.6) (drill 0.3) (layers "F.Cu" "B.Cu") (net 13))
 (segment (start 24.892 51.816) (end 24.892 48.26) (width 0.2) (layer "B.Cu") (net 13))
 (segment (start 25.4 43.688) (end 43.864 43.688) (width 0.2) (layer "B.Cu") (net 13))
 (segment (start 23.876 52.832) (end 24.892 51.816) (width 0.2) (layer "B.Cu") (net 13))
 (segment (start 43.864 43.688) (end 44.792 44.616) (width 0.2) (layer "B.Cu") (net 13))
 (segment (start 19.812 52.832) (end 22.352 52.832) (width 0.2) (layer "B.Cu") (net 13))
 (segment (start 22.352 52.832) (end 23.876 52.832) (width 0.2) (layer "B.Cu") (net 13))
 (segment (start 46.736 61.976) (end 50.292 61.976) (width 0.2) (layer "F.Cu") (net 2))
 (segment (start 50.292 61.976) (end 51.992 60.276) (width 0.2) (layer "F.Cu") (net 2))
 (segment (start 51.992 60.276) (end 51.992 57.912) (width 0.2) (layer "F.Cu") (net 2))
 (via (at 46.736 61.976) (size 0.6) (drill 0.3) (layers "F.Cu" "B.Cu") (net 2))
 (segment (start 51.992 47.752) (end 51.992 45.388) (width 0.2) (layer "B.Cu") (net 2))
 (segment (start 51.992 57.912) (end 51.992 47.752) (width 0.2) (layer "B.Cu") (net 2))
 (segment (start 19.812 58.928) (end 22.352 58.928) (width 0.2) (layer "B.Cu") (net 2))
 (segment (start 22.352 58.928) (end 25.4 61.976) (width 0.2) (layer "B.Cu") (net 2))
 (segment (start 25.4 61.976) (end 46.736 61.976) (width 0.2) (layer "B.Cu") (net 2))
 (segment (start 40.132 42.164) (end 37.9425 39.9745) (width 0.2) (layer "B.Cu") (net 2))
 (segment (start 37.9425 39.9745) (end 37.9425 34.71) (width 0.2) (layer "B.Cu") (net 2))
 (segment (start 48.768 42.164) (end 40.132 42.164) (width 0.2) (layer "B.Cu") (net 2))
 (segment (start 51.992 45.388) (end 48.768 42.164) (width 0.2) (layer "B.Cu") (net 2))
 (segment (start 56.896 63.5) (end 59.192 61.204) (width 0.2) (layer "F.Cu") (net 7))
 (segment (start 59.192 61.204) (end 59.192 57.912) (width 0.2) (layer "F.Cu") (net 7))
 (segment (start 46.736 63.5) (end 56.896 63.5) (width 0.2) (layer "F.Cu") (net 7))
 (via (at 46.736 63.5) (size 0.6) (drill 0.3) (layers "F.Cu" "B.Cu") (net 7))
 (segment (start 19.812 64.516) (end 22.352 64.516) (width 0.2) (layer "B.Cu") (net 7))
 (segment (start 26.416 64.516) (end 27.432 63.5) (width 0.2) (layer "B.Cu") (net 7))
 (segment (start 27.432 63.5) (end 46.736 63.5) (width 0.2) (layer "B.Cu") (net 7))
 (segment (start 59.192 44.968) (end 57.912 43.688) (width 0.2) (layer "B.Cu") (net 7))
 (segment (start 57.912 43.688) (end 54.356 43.688) (width 0.2) (layer "B.Cu") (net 7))
 (segment (start 54.356 43.688) (end 47.9425 37.2745) (width 0.2) (layer "B.Cu") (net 7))
 (segment (start 59.192 57.912) (end 59.192 47.752) (width 0.2) (layer "B.Cu") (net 7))
 (segment (start 59.192 47.752) (end 59.192 44.968) (width 0.2) (layer "B.Cu") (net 7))
 (segment (start 22.352 64.516) (end 26.416 64.516) (width 0.2) (layer "B.Cu") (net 7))
 (segment (start 47.9425 37.2745) (end 47.9425 34.71) (width 0.2) (layer "B.Cu") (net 7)))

